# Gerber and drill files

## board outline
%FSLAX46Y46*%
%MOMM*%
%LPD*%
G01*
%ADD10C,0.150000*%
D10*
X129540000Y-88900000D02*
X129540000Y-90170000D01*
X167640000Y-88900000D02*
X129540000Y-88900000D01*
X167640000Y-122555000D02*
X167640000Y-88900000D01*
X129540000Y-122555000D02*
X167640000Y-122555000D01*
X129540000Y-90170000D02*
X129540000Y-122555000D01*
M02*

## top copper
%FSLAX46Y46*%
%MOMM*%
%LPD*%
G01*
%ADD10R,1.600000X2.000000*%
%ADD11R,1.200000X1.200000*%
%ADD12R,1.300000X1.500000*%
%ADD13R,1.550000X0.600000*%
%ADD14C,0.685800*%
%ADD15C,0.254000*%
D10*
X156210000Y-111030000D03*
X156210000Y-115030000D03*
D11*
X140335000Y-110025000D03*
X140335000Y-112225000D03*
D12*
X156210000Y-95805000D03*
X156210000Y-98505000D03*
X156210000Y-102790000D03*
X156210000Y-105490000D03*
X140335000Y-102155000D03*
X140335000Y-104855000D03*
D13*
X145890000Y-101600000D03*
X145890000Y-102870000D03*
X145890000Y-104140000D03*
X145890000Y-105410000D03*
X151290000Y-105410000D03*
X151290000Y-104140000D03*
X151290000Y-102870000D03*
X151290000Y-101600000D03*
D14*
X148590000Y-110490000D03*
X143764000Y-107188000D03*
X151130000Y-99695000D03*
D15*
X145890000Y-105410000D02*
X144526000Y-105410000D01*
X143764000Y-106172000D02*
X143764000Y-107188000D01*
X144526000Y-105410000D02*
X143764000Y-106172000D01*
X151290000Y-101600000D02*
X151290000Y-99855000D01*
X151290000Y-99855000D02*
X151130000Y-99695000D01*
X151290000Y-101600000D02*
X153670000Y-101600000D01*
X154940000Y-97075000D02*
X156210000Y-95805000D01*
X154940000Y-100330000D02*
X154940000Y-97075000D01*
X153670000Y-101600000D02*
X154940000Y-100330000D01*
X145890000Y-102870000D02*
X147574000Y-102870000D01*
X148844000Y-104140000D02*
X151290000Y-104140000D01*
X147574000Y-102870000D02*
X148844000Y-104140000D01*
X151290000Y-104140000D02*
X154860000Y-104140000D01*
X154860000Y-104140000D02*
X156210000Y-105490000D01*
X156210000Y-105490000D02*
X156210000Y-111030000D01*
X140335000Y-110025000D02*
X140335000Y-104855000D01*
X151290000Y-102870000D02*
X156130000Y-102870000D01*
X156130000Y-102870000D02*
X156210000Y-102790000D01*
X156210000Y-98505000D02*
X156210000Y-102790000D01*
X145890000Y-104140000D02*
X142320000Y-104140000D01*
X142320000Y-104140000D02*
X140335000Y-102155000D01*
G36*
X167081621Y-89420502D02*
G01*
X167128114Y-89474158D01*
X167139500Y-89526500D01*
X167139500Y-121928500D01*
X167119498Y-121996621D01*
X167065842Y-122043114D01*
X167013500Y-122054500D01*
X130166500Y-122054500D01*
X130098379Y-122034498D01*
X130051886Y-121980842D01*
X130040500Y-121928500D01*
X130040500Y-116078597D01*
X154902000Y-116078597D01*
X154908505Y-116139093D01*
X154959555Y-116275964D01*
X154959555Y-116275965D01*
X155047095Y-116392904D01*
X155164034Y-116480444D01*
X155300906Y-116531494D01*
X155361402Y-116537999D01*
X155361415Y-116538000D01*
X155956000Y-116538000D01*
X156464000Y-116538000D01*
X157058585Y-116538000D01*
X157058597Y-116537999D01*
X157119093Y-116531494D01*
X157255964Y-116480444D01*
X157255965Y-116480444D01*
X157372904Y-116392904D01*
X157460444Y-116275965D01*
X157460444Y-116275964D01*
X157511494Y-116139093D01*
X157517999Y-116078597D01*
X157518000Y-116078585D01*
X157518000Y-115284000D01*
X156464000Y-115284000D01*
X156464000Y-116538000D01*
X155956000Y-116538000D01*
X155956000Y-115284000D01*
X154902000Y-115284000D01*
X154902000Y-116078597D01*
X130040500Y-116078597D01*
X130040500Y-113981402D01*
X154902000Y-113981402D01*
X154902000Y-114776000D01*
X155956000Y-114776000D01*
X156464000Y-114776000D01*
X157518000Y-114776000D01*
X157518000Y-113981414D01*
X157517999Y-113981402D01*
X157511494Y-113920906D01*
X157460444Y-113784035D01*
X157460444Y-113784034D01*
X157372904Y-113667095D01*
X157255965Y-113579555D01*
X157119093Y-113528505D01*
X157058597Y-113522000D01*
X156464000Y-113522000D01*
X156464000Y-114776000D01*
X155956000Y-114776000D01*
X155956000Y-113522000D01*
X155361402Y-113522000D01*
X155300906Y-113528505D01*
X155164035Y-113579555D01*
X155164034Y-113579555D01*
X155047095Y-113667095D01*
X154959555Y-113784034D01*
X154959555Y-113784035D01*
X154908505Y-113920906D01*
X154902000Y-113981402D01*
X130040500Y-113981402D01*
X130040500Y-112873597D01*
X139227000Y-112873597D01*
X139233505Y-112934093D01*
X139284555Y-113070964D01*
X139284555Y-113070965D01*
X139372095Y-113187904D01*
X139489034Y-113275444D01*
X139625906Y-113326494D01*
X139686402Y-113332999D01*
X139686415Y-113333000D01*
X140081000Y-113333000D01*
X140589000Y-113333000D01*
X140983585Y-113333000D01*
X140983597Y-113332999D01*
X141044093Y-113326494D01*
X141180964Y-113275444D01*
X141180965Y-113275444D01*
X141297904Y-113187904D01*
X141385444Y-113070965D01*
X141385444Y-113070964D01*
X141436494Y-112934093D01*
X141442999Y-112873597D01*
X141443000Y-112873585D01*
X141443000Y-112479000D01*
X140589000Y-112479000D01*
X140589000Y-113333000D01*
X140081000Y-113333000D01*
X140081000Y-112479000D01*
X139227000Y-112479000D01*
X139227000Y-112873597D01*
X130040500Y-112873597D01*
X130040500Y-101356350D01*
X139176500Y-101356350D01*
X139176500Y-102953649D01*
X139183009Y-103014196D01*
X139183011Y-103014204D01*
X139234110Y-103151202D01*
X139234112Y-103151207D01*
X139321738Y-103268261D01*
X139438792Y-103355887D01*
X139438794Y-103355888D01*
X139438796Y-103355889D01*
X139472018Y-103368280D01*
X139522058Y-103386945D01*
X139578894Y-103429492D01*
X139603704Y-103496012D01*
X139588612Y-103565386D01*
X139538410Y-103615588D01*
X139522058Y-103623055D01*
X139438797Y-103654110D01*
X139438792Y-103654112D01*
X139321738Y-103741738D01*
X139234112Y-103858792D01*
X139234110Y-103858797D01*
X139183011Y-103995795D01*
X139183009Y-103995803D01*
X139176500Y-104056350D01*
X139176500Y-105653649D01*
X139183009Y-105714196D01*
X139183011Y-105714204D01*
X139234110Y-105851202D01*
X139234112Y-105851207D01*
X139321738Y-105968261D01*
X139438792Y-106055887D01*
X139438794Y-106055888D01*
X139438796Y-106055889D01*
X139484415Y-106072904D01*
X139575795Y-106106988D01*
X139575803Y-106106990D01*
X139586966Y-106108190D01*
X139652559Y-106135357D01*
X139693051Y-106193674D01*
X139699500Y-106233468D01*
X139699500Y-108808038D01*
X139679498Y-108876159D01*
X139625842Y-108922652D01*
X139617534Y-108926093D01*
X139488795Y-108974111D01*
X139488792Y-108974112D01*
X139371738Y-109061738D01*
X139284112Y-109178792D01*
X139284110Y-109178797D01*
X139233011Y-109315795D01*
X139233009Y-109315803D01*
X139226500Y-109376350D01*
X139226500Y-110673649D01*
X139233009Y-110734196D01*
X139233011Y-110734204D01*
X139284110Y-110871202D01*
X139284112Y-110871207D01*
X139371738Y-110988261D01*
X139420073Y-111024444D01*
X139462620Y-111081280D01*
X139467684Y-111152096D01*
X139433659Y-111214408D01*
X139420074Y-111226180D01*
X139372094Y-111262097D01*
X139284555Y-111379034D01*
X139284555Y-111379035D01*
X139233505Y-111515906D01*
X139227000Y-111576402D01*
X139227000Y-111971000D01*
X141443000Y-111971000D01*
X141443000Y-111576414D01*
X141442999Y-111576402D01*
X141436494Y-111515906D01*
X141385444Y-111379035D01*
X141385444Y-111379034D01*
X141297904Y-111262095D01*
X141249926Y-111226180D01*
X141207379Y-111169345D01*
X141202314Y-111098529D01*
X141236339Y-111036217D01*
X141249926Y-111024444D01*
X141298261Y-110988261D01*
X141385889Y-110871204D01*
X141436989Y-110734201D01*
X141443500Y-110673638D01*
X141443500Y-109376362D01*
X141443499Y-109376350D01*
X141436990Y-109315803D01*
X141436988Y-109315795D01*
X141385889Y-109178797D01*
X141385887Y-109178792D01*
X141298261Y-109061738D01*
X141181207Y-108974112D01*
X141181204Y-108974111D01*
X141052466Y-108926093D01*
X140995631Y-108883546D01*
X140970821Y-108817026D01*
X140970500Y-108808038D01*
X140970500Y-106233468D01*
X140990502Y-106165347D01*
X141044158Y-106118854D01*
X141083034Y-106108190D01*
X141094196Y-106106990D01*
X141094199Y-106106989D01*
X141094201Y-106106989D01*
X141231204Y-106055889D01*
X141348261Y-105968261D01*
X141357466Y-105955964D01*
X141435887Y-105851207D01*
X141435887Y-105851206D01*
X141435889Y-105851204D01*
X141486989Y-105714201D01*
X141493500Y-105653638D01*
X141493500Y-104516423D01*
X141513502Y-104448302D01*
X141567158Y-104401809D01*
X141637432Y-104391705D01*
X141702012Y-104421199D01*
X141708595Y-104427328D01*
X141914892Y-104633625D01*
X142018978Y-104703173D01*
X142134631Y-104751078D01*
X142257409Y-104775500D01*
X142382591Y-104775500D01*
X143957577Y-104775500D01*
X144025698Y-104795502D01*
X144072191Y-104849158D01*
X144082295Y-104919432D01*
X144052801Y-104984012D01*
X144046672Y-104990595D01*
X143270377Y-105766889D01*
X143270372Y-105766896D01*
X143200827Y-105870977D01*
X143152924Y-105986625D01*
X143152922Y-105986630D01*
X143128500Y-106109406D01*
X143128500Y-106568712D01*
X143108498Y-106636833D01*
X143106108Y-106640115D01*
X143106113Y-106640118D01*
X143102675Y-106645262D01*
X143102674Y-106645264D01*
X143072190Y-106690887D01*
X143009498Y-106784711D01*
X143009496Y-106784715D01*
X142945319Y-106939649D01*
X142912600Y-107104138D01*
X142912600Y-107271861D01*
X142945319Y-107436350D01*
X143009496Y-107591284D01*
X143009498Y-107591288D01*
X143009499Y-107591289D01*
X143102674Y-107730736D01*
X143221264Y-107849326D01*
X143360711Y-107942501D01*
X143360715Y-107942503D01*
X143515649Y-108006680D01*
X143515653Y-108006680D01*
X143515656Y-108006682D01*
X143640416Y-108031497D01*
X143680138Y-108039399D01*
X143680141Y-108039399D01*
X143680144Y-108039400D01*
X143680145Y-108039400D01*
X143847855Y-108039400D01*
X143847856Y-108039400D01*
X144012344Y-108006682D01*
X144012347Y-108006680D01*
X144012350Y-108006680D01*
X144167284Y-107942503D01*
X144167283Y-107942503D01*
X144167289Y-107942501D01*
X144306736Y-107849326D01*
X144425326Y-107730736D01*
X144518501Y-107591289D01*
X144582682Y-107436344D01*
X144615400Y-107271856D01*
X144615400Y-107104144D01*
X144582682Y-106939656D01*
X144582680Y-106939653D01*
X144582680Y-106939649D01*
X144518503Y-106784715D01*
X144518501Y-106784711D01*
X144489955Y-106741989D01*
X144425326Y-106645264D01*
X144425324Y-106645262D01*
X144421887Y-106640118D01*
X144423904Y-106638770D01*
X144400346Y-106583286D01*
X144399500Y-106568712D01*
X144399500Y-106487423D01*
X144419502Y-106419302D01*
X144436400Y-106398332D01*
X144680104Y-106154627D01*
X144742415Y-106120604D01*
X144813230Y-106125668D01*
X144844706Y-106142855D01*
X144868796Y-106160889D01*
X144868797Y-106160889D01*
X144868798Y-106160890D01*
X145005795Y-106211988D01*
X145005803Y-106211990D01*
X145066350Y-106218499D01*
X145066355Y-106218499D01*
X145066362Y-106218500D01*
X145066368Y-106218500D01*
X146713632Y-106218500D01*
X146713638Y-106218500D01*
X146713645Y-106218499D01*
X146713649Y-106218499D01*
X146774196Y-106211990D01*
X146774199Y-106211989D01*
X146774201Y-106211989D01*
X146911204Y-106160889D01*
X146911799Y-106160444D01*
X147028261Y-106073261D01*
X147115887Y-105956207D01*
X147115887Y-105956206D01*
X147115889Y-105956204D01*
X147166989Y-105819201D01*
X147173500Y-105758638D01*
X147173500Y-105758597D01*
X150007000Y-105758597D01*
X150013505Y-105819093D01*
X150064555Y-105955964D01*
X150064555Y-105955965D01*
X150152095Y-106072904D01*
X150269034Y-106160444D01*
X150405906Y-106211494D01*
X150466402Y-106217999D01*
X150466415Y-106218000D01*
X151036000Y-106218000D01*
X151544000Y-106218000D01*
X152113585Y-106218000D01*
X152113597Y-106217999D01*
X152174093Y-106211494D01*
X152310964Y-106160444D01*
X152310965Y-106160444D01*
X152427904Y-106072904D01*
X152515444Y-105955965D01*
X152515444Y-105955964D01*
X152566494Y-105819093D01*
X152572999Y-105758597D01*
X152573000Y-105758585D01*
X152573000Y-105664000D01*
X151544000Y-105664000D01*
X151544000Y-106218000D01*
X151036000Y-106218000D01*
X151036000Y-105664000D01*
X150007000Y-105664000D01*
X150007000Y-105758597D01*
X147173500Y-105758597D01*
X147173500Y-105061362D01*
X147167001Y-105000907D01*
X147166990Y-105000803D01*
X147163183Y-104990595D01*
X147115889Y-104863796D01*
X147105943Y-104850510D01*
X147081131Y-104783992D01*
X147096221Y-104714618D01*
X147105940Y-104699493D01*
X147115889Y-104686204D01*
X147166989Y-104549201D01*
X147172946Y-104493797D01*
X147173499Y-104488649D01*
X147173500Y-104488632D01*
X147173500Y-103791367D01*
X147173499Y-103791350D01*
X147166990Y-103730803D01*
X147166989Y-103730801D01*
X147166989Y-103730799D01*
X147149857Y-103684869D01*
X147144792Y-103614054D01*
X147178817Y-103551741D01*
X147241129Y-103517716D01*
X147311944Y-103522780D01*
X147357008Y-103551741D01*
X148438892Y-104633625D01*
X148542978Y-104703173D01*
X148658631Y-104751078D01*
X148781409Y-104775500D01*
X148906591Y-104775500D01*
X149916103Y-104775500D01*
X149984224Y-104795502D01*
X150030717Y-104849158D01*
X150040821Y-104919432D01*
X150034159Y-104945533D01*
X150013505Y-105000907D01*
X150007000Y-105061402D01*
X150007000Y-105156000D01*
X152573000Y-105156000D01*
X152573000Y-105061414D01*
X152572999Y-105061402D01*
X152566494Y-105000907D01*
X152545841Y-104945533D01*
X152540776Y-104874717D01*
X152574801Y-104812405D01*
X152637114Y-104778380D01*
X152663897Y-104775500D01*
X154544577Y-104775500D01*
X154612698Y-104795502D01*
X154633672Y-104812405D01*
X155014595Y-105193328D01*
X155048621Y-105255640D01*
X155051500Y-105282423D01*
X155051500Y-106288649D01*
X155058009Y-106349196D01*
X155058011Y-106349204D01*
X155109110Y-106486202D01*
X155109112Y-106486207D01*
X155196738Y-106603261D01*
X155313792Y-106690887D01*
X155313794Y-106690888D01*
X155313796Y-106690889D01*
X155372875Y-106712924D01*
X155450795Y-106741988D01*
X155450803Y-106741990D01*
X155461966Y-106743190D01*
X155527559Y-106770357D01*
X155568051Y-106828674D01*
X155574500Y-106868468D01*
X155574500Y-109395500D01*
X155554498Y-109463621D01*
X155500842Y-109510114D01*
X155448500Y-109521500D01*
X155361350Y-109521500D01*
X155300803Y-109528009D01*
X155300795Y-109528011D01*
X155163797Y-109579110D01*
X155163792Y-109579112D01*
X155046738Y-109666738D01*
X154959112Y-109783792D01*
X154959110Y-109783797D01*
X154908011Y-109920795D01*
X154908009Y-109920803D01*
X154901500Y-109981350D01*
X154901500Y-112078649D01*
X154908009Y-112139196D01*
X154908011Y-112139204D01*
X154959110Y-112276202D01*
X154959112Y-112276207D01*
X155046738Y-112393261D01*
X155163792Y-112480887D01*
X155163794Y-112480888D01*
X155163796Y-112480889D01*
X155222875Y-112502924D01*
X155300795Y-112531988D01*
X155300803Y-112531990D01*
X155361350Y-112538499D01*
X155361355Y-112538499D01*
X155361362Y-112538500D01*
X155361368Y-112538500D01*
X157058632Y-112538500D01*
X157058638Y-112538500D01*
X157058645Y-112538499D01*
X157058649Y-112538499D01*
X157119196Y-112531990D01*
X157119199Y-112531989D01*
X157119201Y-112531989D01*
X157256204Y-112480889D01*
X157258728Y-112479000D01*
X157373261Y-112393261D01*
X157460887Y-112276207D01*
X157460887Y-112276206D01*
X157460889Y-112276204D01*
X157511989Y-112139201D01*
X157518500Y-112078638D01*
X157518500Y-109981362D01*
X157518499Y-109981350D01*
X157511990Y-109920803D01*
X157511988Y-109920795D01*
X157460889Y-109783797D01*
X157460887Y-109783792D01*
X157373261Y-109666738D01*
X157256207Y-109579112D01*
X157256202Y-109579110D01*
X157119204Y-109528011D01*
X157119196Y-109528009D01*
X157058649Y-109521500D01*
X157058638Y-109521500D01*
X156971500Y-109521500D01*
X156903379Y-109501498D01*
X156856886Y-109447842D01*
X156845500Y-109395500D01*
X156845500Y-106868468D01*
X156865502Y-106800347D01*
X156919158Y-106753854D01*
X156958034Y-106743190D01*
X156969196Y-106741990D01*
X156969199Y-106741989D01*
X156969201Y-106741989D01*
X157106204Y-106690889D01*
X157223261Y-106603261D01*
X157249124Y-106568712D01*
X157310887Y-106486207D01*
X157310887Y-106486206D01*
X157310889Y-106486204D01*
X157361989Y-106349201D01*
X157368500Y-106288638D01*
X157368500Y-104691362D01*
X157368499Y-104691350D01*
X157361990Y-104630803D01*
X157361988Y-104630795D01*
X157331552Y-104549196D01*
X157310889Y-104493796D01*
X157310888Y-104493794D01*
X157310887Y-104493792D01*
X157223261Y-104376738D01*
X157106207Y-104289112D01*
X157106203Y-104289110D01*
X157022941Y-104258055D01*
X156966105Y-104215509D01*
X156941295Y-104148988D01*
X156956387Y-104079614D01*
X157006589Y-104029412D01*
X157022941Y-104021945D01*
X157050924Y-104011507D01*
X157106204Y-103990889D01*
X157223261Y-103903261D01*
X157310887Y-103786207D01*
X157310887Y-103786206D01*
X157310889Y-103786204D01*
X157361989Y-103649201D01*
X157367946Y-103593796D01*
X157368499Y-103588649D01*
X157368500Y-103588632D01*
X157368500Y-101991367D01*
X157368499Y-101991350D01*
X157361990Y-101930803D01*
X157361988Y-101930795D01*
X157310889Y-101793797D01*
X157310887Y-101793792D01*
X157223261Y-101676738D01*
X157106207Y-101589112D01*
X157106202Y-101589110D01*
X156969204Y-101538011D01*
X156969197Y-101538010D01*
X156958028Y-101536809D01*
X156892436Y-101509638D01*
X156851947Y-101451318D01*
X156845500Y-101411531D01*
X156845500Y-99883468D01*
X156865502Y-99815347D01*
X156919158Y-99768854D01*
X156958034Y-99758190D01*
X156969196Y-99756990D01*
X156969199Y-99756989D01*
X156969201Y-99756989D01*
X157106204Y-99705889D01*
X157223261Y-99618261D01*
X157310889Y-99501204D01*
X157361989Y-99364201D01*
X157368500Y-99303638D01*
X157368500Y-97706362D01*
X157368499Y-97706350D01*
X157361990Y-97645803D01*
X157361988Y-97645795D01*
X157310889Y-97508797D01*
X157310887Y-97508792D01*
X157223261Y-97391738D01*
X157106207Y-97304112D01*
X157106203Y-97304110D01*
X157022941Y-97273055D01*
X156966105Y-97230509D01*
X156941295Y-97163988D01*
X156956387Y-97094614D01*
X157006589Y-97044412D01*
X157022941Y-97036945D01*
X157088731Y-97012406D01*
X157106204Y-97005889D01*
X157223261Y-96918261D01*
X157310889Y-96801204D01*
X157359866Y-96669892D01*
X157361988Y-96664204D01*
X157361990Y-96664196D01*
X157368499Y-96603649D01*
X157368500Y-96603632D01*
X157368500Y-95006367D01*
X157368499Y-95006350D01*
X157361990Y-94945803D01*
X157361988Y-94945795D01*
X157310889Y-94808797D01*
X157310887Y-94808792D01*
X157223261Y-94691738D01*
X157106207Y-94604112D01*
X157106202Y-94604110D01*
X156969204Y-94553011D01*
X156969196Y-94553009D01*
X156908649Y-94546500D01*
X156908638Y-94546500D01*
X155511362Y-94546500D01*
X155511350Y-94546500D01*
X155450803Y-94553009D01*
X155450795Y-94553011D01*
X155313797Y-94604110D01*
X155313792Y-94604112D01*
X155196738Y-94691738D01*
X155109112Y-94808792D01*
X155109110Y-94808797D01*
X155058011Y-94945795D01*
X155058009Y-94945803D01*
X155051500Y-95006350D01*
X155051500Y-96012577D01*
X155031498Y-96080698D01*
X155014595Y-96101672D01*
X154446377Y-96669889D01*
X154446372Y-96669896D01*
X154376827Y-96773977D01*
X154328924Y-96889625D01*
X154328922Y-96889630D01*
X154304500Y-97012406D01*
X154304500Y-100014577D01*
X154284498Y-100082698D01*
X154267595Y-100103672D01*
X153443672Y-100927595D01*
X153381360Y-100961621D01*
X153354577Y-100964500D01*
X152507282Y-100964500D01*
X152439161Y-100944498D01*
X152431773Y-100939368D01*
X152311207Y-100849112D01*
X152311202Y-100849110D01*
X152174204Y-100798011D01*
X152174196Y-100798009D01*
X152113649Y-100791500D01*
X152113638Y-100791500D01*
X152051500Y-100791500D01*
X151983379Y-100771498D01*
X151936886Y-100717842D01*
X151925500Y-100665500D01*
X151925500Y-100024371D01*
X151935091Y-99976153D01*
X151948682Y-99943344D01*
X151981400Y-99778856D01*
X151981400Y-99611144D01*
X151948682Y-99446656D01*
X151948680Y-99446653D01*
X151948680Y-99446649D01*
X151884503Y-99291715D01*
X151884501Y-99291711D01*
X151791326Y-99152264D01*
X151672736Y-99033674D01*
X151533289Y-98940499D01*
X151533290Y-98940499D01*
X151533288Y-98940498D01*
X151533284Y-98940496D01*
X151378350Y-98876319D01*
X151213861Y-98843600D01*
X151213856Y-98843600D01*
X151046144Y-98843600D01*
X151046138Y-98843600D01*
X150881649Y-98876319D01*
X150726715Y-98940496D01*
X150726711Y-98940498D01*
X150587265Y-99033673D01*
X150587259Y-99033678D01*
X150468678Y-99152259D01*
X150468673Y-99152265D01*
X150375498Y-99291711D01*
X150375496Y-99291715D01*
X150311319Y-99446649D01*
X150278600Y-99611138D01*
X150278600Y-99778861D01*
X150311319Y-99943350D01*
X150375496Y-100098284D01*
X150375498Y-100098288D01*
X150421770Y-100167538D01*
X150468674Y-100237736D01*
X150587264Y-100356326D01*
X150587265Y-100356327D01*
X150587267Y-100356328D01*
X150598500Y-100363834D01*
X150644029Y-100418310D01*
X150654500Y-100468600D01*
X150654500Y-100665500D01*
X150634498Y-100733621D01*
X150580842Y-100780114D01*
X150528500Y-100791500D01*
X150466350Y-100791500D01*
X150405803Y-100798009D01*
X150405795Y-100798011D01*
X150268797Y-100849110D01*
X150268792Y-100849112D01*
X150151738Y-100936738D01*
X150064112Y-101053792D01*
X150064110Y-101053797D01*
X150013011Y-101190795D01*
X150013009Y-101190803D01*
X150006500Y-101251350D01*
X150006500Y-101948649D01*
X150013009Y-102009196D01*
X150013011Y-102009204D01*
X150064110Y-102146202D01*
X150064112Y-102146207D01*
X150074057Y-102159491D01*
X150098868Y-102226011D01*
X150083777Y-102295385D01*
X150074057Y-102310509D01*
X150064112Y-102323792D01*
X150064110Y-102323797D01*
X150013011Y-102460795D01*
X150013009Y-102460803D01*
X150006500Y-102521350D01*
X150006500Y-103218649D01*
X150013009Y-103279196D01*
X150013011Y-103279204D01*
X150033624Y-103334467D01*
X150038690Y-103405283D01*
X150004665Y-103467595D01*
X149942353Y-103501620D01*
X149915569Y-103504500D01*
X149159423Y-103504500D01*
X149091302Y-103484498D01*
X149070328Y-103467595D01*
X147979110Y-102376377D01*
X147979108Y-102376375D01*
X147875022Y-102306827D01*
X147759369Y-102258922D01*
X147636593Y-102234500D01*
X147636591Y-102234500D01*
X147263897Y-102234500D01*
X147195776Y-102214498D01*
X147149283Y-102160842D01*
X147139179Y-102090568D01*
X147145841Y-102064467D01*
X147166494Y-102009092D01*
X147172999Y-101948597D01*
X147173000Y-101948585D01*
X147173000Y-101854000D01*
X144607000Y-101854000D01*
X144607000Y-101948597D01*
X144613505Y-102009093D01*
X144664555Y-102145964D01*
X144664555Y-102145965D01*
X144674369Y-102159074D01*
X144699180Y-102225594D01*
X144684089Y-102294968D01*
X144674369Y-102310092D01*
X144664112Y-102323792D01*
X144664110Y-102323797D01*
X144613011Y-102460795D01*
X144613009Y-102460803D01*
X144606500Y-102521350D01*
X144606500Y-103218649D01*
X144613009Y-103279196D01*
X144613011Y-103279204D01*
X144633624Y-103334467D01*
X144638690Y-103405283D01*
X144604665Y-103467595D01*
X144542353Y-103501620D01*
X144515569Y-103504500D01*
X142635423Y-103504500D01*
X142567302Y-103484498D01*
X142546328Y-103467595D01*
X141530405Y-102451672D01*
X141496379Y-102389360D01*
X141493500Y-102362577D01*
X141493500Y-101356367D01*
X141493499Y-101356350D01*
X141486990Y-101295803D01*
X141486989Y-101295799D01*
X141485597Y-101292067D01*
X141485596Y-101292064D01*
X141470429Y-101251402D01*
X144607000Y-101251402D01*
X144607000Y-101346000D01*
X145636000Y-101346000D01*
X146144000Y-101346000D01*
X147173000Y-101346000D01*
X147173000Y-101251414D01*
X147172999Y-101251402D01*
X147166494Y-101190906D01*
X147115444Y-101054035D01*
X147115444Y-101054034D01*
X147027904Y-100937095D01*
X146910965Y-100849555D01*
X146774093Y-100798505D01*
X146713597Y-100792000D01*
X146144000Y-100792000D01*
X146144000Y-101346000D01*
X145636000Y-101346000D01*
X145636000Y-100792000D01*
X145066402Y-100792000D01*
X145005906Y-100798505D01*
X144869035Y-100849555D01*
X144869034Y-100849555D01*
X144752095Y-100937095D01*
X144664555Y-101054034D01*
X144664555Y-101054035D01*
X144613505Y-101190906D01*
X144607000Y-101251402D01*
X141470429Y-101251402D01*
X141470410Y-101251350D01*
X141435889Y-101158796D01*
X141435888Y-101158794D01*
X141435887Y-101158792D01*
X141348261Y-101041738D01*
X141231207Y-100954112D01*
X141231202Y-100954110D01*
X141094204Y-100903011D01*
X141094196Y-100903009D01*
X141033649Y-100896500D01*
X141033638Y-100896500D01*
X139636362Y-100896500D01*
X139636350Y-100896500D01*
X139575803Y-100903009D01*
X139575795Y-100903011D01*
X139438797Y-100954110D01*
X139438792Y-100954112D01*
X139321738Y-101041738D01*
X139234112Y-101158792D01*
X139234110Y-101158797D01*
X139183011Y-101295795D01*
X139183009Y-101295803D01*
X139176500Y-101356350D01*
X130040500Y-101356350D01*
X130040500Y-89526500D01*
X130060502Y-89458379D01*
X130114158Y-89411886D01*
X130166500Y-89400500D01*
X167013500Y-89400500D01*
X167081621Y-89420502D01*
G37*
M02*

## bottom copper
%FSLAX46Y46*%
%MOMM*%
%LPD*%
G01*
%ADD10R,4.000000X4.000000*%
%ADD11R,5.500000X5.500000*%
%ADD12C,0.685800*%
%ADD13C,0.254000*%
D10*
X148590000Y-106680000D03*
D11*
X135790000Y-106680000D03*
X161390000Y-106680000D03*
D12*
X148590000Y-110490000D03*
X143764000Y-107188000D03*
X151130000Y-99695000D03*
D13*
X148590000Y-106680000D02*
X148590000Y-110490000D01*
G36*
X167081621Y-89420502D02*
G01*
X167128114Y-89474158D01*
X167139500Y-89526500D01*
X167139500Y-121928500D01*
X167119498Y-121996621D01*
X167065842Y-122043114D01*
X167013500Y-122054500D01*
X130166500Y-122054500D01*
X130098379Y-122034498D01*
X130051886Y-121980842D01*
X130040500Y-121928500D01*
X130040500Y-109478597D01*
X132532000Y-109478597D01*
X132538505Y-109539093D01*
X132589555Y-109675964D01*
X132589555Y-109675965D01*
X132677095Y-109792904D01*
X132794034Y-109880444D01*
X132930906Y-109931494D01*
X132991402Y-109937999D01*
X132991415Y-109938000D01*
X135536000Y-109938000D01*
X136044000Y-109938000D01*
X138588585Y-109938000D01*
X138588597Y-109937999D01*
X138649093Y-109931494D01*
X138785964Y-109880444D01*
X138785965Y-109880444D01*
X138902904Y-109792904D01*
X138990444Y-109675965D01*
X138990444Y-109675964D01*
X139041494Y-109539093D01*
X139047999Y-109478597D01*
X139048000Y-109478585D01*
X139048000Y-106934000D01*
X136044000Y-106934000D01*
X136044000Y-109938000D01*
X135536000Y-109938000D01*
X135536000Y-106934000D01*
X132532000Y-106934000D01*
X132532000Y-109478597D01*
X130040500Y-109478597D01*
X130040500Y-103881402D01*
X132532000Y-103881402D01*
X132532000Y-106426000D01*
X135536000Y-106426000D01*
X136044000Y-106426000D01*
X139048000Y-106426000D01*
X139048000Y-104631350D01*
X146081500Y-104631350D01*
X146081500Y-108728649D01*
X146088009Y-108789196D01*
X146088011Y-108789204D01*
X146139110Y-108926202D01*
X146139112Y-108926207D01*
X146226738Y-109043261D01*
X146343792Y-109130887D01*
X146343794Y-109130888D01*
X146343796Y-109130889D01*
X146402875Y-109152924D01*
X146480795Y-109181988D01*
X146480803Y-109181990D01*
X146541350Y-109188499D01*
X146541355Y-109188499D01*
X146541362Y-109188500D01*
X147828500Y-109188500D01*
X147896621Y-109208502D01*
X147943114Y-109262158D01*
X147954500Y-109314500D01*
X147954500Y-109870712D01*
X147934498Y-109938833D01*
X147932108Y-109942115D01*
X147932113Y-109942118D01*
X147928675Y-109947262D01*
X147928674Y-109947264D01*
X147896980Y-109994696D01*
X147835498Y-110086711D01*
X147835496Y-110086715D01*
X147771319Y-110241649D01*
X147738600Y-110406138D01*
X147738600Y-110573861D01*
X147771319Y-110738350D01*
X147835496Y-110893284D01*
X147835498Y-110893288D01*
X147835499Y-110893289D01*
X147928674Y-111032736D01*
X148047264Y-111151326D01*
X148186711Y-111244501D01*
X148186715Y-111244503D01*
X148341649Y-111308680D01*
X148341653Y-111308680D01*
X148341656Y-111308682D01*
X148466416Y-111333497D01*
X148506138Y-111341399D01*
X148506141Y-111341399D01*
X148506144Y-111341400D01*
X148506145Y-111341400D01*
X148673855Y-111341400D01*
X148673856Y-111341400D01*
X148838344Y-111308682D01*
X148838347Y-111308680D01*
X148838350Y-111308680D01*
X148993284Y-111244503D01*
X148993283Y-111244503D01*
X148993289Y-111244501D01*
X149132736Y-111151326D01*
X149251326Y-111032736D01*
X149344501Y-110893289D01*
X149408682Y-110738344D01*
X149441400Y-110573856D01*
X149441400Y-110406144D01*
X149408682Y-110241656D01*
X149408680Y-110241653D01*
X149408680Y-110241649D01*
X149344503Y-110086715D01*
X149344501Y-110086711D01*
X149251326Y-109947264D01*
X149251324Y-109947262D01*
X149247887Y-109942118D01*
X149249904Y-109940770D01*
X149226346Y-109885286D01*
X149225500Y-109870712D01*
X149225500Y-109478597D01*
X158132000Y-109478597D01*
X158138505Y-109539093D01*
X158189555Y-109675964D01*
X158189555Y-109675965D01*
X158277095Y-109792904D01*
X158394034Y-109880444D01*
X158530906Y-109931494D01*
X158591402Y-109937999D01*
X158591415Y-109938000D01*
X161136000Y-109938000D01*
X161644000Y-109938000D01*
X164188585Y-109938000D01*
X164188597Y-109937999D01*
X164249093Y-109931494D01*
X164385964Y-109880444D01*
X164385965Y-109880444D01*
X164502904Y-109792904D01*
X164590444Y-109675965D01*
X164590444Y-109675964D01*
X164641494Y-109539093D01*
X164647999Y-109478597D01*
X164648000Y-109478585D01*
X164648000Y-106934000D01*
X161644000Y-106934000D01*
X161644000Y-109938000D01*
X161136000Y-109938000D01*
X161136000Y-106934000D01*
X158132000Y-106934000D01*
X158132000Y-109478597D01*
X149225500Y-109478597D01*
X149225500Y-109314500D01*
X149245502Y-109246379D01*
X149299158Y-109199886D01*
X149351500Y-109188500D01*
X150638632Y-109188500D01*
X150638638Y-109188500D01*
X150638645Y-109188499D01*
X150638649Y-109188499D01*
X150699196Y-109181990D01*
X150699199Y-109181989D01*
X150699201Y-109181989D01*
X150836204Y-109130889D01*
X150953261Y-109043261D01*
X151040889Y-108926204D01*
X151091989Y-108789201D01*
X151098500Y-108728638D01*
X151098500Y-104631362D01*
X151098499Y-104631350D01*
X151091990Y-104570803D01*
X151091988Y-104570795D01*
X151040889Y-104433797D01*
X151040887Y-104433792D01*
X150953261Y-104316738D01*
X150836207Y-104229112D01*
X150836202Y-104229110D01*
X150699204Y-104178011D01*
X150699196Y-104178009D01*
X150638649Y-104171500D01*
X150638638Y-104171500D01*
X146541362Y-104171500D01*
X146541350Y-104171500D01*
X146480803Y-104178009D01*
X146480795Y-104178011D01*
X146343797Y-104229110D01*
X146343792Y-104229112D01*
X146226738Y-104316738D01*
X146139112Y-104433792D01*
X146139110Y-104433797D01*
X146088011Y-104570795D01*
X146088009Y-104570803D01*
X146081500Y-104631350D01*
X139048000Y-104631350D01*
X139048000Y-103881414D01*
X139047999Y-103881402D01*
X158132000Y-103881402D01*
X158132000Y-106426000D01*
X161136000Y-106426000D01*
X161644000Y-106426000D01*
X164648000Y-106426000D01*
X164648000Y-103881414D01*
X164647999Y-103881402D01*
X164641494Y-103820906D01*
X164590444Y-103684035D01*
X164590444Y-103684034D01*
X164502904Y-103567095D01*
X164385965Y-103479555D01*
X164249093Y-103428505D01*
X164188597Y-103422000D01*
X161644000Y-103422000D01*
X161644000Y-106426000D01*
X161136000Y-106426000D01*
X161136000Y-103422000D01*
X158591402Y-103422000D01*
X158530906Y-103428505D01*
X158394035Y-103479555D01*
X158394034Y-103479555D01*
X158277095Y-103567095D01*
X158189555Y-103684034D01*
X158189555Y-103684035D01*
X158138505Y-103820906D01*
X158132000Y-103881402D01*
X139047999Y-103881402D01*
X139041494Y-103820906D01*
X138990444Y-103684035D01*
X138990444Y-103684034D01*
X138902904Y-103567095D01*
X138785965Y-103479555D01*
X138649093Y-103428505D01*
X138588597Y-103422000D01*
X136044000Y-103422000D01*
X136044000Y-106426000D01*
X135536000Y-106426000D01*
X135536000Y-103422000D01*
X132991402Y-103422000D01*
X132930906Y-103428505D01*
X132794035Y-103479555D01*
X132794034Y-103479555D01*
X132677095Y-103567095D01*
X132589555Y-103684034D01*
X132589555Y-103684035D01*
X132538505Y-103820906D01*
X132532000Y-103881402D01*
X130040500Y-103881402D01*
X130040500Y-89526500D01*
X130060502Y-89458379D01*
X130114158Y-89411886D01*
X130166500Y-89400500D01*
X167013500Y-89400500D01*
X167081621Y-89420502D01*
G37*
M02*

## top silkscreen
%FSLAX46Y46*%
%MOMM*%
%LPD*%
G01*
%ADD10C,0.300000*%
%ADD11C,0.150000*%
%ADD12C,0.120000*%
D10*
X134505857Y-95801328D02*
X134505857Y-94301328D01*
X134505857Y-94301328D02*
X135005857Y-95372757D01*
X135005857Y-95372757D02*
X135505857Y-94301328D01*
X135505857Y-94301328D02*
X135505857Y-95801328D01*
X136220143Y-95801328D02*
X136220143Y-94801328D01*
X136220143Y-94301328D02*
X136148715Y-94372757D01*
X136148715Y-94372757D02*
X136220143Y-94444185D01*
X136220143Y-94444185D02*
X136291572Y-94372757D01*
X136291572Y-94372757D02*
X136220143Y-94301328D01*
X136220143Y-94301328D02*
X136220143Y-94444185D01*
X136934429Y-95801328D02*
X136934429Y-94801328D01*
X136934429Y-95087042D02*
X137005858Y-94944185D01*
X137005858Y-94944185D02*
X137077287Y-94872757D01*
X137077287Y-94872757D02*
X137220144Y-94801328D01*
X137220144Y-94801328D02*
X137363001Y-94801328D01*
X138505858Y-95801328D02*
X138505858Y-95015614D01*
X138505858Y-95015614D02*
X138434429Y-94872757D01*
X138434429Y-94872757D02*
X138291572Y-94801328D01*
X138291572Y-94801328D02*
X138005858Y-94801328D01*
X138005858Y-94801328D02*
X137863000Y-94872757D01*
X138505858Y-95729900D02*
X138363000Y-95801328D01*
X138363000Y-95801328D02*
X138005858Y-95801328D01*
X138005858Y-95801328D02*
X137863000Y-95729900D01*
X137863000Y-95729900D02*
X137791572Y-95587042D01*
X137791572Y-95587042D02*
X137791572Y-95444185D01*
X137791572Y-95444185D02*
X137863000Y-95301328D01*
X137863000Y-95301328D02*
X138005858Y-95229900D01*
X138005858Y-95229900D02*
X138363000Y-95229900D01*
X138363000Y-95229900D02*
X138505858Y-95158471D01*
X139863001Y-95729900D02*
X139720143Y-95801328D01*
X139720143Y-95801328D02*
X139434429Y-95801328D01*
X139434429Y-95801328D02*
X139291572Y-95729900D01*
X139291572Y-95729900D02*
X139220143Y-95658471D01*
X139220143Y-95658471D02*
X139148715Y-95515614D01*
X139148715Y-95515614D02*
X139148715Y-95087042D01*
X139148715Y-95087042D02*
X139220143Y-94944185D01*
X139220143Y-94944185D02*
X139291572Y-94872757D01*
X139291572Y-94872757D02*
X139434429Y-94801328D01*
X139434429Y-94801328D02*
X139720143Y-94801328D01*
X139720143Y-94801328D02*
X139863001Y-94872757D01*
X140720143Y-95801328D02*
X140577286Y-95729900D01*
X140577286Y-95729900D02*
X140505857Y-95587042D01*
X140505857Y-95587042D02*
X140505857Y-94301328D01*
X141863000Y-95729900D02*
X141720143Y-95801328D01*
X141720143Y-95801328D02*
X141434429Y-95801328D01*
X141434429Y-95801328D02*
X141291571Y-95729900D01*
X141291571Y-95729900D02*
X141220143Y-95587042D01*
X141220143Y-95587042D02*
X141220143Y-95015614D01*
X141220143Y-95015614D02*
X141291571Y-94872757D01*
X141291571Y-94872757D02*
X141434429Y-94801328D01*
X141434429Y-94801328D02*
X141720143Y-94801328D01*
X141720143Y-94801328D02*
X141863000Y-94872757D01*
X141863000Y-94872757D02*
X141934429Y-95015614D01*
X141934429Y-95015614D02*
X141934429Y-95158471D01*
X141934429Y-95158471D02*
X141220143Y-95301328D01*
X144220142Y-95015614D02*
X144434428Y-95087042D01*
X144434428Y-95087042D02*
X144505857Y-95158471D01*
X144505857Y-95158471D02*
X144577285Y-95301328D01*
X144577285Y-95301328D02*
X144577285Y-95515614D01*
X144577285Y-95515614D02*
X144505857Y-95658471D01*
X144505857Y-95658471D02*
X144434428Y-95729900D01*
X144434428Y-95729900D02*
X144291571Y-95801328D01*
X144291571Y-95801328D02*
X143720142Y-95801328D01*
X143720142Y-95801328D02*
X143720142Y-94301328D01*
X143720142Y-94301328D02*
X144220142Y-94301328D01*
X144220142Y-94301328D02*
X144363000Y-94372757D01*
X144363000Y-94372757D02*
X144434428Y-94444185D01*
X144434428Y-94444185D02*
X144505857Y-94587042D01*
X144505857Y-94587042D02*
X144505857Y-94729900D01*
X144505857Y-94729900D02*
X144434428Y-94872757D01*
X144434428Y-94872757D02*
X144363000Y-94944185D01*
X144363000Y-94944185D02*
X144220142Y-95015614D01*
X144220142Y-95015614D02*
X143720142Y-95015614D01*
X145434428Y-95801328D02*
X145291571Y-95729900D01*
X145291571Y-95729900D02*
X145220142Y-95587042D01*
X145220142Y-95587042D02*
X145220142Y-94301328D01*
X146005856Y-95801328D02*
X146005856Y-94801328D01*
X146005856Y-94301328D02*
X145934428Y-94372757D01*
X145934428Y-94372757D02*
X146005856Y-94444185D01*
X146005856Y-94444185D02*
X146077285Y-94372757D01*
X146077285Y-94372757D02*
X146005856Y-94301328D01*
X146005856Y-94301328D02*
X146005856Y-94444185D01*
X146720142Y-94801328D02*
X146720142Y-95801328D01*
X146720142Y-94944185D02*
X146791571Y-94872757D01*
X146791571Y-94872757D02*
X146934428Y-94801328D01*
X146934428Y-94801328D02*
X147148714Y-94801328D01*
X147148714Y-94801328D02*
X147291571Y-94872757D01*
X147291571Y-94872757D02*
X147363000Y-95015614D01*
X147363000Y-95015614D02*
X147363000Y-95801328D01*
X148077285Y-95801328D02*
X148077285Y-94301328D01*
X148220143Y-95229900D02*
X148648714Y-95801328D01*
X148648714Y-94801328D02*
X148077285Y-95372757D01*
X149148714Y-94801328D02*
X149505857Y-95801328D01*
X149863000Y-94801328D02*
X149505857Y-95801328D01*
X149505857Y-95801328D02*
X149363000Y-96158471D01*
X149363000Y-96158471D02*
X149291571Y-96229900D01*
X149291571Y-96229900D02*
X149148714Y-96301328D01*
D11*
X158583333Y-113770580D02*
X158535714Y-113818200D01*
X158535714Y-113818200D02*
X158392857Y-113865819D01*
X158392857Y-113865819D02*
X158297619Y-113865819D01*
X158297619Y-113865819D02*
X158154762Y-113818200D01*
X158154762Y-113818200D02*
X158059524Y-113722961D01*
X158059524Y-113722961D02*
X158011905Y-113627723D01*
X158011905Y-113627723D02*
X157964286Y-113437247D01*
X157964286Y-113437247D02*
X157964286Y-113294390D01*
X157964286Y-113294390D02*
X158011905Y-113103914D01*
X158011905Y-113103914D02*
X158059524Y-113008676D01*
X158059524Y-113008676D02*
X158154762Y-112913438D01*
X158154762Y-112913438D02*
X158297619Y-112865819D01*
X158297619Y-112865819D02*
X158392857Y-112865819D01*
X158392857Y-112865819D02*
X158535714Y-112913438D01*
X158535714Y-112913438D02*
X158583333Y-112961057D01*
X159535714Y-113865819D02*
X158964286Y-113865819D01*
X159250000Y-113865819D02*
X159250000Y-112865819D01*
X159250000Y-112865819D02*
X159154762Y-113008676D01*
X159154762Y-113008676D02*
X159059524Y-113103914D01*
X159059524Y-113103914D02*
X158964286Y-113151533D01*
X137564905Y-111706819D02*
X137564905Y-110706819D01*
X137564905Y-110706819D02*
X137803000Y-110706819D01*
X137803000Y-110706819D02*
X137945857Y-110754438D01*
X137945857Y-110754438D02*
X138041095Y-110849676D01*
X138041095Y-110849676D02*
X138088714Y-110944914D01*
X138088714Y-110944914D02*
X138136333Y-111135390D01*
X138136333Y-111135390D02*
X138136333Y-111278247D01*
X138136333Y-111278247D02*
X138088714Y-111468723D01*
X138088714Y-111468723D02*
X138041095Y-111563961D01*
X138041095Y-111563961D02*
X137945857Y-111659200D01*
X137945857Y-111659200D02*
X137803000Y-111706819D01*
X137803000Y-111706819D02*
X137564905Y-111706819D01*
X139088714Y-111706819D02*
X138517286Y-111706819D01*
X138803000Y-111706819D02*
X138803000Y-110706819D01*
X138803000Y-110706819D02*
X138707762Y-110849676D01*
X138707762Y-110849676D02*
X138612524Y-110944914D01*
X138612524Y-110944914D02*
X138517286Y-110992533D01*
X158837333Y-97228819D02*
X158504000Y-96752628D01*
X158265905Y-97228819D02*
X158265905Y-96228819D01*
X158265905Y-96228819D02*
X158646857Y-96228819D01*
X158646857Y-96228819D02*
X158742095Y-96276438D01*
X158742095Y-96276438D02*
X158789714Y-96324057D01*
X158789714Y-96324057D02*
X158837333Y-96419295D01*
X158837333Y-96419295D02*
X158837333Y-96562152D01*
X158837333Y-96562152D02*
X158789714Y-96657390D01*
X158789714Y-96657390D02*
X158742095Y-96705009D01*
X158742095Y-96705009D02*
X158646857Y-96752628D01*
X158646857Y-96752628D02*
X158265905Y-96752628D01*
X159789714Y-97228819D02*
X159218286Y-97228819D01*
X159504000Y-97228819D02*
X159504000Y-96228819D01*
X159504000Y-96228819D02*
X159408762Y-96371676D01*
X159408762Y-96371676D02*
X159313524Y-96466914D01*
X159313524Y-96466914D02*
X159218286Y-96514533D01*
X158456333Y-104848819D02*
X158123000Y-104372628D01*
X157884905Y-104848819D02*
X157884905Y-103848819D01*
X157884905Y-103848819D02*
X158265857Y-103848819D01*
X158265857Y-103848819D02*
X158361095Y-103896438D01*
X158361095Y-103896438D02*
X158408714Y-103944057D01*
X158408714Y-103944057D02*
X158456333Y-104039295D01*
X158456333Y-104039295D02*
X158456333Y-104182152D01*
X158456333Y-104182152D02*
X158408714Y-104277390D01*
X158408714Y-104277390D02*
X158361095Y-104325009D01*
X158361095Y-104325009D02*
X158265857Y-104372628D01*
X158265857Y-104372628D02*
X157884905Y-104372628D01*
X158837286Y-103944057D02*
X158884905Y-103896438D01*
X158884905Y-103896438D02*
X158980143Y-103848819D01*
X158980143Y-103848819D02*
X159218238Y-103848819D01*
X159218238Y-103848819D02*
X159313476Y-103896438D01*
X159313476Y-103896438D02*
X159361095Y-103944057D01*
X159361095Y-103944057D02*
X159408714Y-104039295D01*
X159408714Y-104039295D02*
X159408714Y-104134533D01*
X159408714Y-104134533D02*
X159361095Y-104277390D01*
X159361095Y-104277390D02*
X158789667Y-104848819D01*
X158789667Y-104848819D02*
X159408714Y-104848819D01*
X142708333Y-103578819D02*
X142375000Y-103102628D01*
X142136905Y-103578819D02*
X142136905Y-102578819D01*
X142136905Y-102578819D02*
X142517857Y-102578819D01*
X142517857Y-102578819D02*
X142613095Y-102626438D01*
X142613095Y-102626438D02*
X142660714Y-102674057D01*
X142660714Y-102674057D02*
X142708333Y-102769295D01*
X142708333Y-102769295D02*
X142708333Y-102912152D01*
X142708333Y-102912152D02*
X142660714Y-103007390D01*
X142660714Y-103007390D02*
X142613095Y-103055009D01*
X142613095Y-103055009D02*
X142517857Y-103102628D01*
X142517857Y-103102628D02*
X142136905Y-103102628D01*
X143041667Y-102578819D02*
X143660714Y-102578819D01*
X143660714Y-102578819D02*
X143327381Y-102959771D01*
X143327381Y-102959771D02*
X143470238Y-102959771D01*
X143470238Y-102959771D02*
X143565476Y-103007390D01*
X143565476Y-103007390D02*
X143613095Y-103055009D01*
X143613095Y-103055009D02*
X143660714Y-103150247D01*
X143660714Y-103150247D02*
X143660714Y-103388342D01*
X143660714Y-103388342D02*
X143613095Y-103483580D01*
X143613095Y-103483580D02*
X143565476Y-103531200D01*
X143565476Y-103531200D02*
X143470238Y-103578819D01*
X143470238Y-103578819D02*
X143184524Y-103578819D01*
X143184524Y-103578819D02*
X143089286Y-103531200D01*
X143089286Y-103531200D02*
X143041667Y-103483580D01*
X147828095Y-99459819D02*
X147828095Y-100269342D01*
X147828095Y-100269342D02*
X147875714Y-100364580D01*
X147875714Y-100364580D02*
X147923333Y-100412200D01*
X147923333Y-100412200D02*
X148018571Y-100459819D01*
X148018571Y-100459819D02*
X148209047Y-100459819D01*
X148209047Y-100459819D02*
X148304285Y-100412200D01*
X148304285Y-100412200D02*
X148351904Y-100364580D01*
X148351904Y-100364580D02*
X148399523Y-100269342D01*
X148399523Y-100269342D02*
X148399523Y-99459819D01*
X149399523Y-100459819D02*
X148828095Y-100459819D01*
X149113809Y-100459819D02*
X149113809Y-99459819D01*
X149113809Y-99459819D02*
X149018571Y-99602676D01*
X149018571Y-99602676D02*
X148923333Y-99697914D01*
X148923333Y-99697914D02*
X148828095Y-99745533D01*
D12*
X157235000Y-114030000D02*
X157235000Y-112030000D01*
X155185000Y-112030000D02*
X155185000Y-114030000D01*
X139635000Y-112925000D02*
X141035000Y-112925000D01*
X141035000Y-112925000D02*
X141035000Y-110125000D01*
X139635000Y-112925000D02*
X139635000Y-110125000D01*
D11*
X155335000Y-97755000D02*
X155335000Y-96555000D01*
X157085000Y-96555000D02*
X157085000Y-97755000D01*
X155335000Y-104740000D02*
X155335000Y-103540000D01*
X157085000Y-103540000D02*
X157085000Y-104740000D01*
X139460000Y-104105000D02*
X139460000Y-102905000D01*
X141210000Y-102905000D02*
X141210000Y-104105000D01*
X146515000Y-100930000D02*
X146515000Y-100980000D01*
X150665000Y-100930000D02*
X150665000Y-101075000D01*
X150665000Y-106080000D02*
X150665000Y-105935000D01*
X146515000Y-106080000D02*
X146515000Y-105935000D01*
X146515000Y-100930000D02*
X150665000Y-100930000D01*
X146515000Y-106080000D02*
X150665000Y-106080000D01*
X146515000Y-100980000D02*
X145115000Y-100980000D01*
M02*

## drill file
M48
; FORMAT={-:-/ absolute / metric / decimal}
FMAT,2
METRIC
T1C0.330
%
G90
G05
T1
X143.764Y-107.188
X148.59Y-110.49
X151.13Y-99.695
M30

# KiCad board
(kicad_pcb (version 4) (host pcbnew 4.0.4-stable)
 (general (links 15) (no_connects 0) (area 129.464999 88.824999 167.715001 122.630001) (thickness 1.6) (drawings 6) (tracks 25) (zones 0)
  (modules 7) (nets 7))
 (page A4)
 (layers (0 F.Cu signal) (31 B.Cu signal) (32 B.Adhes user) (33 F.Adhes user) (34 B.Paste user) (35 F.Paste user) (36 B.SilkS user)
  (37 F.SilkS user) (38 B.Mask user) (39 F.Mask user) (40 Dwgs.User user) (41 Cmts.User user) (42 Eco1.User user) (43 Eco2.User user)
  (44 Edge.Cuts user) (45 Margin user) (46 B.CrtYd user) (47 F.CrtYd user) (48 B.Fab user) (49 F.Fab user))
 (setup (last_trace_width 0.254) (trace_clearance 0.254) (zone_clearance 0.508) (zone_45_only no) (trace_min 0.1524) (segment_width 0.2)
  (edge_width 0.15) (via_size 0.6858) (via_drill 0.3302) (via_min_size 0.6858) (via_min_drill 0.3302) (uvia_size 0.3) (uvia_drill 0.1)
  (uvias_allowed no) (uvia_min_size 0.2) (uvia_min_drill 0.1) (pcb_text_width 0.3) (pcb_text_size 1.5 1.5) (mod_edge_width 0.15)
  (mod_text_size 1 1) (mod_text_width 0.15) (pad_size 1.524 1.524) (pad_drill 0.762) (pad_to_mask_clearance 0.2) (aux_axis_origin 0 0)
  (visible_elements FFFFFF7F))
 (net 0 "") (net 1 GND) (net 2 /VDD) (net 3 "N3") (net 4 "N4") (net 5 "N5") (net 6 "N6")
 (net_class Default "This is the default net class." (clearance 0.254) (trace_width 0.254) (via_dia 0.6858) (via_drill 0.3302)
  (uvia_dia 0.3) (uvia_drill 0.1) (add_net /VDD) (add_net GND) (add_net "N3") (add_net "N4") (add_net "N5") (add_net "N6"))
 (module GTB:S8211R (layer B.Cu) (at 148.59 106.68)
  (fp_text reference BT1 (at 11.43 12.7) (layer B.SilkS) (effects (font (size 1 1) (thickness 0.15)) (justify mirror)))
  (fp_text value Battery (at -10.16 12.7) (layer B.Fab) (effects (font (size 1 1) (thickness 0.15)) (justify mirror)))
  (pad 2 smd rect (at 0 0) (size 4 4) (layers B.Cu B.Paste B.Mask) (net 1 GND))
  (pad 1 smd rect (at -12.8 0) (size 5.5 5.5) (layers B.Cu B.Paste B.Mask) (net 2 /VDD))
  (pad 1 smd rect (at 12.8 0) (size 5.5 5.5) (layers B.Cu B.Paste B.Mask) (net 2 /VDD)))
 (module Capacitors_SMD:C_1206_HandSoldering (layer F.Cu) (at 156.21 113.03 270)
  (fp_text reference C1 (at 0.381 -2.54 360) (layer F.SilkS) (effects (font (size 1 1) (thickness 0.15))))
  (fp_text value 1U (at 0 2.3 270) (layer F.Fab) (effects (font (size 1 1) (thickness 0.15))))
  (fp_line (start 1 -1.025) (end -1 -1.025) (layer F.SilkS) (width 0.12))
  (fp_line (start -1 1.025) (end 1 1.025) (layer F.SilkS) (width 0.12))
  (pad 1 smd rect (at -2 0 270) (size 2 1.6) (layers F.Cu F.Paste F.Mask) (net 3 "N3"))
  (pad 2 smd rect (at 2 0 270) (size 2 1.6) (layers F.Cu F.Paste F.Mask) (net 1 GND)))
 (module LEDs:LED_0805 (layer F.Cu) (at 140.335 111.125 90)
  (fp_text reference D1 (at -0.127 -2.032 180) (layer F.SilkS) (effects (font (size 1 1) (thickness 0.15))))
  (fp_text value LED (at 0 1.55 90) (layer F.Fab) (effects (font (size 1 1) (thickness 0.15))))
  (fp_line (start -1.8 -0.7) (end -1.8 0.7) (layer F.SilkS) (width 0.12))
  (fp_line (start -1.8 0.7) (end 1 0.7) (layer F.SilkS) (width 0.12))
  (fp_line (start -1.8 -0.7) (end 1 -0.7) (layer F.SilkS) (width 0.12))
  (pad 2 smd rect (at 1.1 0 270) (size 1.2 1.2) (layers F.Cu F.Paste F.Mask) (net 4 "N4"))
  (pad 1 smd rect (at -1.1 0 270) (size 1.2 1.2) (layers F.Cu F.Paste F.Mask) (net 1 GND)))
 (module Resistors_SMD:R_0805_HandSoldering (layer F.Cu) (at 156.21 97.155 270)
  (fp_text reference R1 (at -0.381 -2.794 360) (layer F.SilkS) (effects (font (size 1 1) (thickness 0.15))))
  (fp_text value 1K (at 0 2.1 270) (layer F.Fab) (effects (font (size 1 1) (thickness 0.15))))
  (fp_line (start 0.6 0.875) (end -0.6 0.875) (layer F.SilkS) (width 0.15))
  (fp_line (start -0.6 -0.875) (end 0.6 -0.875) (layer F.SilkS) (width 0.15))
  (pad 1 smd rect (at -1.35 0 270) (size 1.5 1.3) (layers F.Cu F.Paste F.Mask) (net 2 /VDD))
  (pad 2 smd rect (at 1.35 0 270) (size 1.5 1.3) (layers F.Cu F.Paste F.Mask) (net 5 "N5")))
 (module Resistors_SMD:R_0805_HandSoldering (layer F.Cu) (at 156.21 104.14 270)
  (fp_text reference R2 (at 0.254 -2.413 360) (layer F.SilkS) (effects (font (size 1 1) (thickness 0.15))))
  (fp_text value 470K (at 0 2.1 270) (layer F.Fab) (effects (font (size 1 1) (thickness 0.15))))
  (fp_line (start 0.6 0.875) (end -0.6 0.875) (layer F.SilkS) (width 0.15))
  (fp_line (start -0.6 -0.875) (end 0.6 -0.875) (layer F.SilkS) (width 0.15))
  (pad 1 smd rect (at -1.35 0 270) (size 1.5 1.3) (layers F.Cu F.Paste F.Mask) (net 5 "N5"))
  (pad 2 smd rect (at 1.35 0 270) (size 1.5 1.3) (layers F.Cu F.Paste F.Mask) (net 3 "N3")))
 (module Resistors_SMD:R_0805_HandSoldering (layer F.Cu) (at 140.335 103.505 270)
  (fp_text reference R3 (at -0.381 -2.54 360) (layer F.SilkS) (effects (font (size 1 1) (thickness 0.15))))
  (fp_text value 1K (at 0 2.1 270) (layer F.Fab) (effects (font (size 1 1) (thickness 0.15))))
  (fp_line (start 0.6 0.875) (end -0.6 0.875) (layer F.SilkS) (width 0.15))
  (fp_line (start -0.6 -0.875) (end 0.6 -0.875) (layer F.SilkS) (width 0.15))
  (pad 1 smd rect (at -1.35 0 270) (size 1.5 1.3) (layers F.Cu F.Paste F.Mask) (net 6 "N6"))
  (pad 2 smd rect (at 1.35 0 270) (size 1.5 1.3) (layers F.Cu F.Paste F.Mask) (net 4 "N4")))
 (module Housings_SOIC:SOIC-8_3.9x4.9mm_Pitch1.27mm (layer F.Cu) (at 148.59 103.505)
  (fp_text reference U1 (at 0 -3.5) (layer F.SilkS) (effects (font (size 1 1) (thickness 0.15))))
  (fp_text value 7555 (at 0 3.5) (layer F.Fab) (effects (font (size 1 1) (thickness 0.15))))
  (fp_line (start -2.075 -2.575) (end -2.075 -2.525) (layer F.SilkS) (width 0.15))
  (fp_line (start 2.075 -2.575) (end 2.075 -2.43) (layer F.SilkS) (width 0.15))
  (fp_line (start 2.075 2.575) (end 2.075 2.43) (layer F.SilkS) (width 0.15))
  (fp_line (start -2.075 2.575) (end -2.075 2.43) (layer F.SilkS) (width 0.15))
  (fp_line (start -2.075 -2.575) (end 2.075 -2.575) (layer F.SilkS) (width 0.15))
  (fp_line (start -2.075 2.575) (end 2.075 2.575) (layer F.SilkS) (width 0.15))
  (fp_line (start -2.075 -2.525) (end -3.475 -2.525) (layer F.SilkS) (width 0.15))
  (pad 1 smd rect (at -2.7 -1.905) (size 1.55 0.6) (layers F.Cu F.Paste F.Mask) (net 1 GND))
  (pad 2 smd rect (at -2.7 -0.635) (size 1.55 0.6) (layers F.Cu F.Paste F.Mask) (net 3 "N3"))
  (pad 3 smd rect (at -2.7 0.635) (size 1.55 0.6) (layers F.Cu F.Paste F.Mask) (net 6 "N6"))
  (pad 4 smd rect (at -2.7 1.905) (size 1.55 0.6) (layers F.Cu F.Paste F.Mask) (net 2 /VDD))
  (pad 5 smd rect (at 2.7 1.905) (size 1.55 0.6) (layers F.Cu F.Paste F.Mask) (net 1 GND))
  (pad 6 smd rect (at 2.7 0.635) (size 1.55 0.6) (layers F.Cu F.Paste F.Mask) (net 3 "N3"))
  (pad 7 smd rect (at 2.7 -0.635) (size 1.55 0.6) (layers F.Cu F.Paste F.Mask) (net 5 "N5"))
  (pad 8 smd rect (at 2.7 -1.905) (size 1.55 0.6) (layers F.Cu F.Paste F.Mask) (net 2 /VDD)))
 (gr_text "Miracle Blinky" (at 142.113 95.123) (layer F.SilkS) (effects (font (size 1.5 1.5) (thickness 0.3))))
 (gr_line (start 129.54 88.9) (end 129.54 90.17) (angle 90) (layer Edge.Cuts) (width 0.15))
 (gr_line (start 167.64 88.9) (end 129.54 88.9) (angle 90) (layer Edge.Cuts) (width 0.15))
 (gr_line (start 167.64 122.555) (end 167.64 88.9) (angle 90) (layer Edge.Cuts) (width 0.15))
 (gr_line (start 129.54 122.555) (end 167.64 122.555) (angle 90) (layer Edge.Cuts) (width 0.15))
 (gr_line (start 129.54 90.17) (end 129.54 122.555) (angle 90) (layer Edge.Cuts) (width 0.15))
 (segment (start 148.59 106.68) (end 148.59 110.49) (width 0.254) (layer B.Cu) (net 1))
 (via (at 148.59 110.49) (size 0.6858) (drill 0.3302) (layers F.Cu B.Cu) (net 1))
 (segment (start 145.89 105.41) (end 144.526 105.41) (width 0.254) (layer F.Cu) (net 2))
 (via (at 143.764 107.188) (size 0.6858) (drill 0.3302) (layers F.Cu B.Cu) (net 2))
 (segment (start 143.764 106.172) (end 143.764 107.188) (width 0.254) (layer F.Cu) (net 2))
 (segment (start 144.526 105.41) (end 143.764 106.172) (width 0.254) (layer F.Cu) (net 2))
 (segment (start 151.29 101.6) (end 151.29 99.855) (width 0.254) (layer F.Cu) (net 2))
 (via (at 151.13 99.695) (size 0.6858) (drill 0.3302) (layers F.Cu B.Cu) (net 2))
 (segment (start 151.29 99.855) (end 151.13 99.695) (width 0.254) (layer F.Cu) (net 2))
 (segment (start 151.29 101.6) (end 153.67 101.6) (width 0.254) (layer F.Cu) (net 2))
 (segment (start 154.94 97.075) (end 156.21 95.805) (width 0.254) (layer F.Cu) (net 2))
 (segment (start 154.94 100.33) (end 154.94 97.075) (width 0.254) (layer F.Cu) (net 2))
 (segment (start 153.67 101.6) (end 154.94 100.33) (width 0.254) (layer F.Cu) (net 2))
 (segment (start 145.89 102.87) (end 147.574 102.87) (width 0.254) (layer F.Cu) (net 3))
 (segment (start 148.844 104.14) (end 151.29 104.14) (width 0.254) (layer F.Cu) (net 3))
 (segment (start 147.574 102.87) (end 148.844 104.14) (width 0.254) (layer F.Cu) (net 3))
 (segment (start 151.29 104.14) (end 154.86 104.14) (width 0.254) (layer F.Cu) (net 3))
 (segment (start 154.86 104.14) (end 156.21 105.49) (width 0.254) (layer F.Cu) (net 3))
 (segment (start 156.21 105.49) (end 156.21 111.03) (width 0.254) (layer F.Cu) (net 3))
 (segment (start 140.335 110.025) (end 140.335 104.855) (width 0.254) (layer F.Cu) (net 4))
 (segment (start 151.29 102.87) (end 156.13 102.87) (width 0.254) (layer F.Cu) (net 5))
 (segment (start 156.13 102.87) (end 156.21 102.79) (width 0.254) (layer F.Cu) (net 5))
 (segment (start 156.21 98.505) (end 156.21 102.79) (width 0.254) (layer F.Cu) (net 5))
 (segment (start 145.89 104.14) (end 142.32 104.14) (width 0.254) (layer F.Cu) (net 6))
 (segment (start 142.32 104.14) (end 140.335 102.155) (width 0.254) (layer F.Cu) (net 6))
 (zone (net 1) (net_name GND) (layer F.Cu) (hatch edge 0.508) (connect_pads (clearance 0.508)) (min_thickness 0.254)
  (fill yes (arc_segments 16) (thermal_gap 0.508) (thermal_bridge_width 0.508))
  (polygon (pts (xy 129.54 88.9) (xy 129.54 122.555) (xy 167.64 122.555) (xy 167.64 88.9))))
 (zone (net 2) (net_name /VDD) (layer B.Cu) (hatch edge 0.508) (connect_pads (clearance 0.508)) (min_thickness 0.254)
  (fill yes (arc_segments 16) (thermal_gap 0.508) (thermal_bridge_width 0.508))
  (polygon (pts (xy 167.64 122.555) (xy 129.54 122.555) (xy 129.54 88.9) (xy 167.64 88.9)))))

